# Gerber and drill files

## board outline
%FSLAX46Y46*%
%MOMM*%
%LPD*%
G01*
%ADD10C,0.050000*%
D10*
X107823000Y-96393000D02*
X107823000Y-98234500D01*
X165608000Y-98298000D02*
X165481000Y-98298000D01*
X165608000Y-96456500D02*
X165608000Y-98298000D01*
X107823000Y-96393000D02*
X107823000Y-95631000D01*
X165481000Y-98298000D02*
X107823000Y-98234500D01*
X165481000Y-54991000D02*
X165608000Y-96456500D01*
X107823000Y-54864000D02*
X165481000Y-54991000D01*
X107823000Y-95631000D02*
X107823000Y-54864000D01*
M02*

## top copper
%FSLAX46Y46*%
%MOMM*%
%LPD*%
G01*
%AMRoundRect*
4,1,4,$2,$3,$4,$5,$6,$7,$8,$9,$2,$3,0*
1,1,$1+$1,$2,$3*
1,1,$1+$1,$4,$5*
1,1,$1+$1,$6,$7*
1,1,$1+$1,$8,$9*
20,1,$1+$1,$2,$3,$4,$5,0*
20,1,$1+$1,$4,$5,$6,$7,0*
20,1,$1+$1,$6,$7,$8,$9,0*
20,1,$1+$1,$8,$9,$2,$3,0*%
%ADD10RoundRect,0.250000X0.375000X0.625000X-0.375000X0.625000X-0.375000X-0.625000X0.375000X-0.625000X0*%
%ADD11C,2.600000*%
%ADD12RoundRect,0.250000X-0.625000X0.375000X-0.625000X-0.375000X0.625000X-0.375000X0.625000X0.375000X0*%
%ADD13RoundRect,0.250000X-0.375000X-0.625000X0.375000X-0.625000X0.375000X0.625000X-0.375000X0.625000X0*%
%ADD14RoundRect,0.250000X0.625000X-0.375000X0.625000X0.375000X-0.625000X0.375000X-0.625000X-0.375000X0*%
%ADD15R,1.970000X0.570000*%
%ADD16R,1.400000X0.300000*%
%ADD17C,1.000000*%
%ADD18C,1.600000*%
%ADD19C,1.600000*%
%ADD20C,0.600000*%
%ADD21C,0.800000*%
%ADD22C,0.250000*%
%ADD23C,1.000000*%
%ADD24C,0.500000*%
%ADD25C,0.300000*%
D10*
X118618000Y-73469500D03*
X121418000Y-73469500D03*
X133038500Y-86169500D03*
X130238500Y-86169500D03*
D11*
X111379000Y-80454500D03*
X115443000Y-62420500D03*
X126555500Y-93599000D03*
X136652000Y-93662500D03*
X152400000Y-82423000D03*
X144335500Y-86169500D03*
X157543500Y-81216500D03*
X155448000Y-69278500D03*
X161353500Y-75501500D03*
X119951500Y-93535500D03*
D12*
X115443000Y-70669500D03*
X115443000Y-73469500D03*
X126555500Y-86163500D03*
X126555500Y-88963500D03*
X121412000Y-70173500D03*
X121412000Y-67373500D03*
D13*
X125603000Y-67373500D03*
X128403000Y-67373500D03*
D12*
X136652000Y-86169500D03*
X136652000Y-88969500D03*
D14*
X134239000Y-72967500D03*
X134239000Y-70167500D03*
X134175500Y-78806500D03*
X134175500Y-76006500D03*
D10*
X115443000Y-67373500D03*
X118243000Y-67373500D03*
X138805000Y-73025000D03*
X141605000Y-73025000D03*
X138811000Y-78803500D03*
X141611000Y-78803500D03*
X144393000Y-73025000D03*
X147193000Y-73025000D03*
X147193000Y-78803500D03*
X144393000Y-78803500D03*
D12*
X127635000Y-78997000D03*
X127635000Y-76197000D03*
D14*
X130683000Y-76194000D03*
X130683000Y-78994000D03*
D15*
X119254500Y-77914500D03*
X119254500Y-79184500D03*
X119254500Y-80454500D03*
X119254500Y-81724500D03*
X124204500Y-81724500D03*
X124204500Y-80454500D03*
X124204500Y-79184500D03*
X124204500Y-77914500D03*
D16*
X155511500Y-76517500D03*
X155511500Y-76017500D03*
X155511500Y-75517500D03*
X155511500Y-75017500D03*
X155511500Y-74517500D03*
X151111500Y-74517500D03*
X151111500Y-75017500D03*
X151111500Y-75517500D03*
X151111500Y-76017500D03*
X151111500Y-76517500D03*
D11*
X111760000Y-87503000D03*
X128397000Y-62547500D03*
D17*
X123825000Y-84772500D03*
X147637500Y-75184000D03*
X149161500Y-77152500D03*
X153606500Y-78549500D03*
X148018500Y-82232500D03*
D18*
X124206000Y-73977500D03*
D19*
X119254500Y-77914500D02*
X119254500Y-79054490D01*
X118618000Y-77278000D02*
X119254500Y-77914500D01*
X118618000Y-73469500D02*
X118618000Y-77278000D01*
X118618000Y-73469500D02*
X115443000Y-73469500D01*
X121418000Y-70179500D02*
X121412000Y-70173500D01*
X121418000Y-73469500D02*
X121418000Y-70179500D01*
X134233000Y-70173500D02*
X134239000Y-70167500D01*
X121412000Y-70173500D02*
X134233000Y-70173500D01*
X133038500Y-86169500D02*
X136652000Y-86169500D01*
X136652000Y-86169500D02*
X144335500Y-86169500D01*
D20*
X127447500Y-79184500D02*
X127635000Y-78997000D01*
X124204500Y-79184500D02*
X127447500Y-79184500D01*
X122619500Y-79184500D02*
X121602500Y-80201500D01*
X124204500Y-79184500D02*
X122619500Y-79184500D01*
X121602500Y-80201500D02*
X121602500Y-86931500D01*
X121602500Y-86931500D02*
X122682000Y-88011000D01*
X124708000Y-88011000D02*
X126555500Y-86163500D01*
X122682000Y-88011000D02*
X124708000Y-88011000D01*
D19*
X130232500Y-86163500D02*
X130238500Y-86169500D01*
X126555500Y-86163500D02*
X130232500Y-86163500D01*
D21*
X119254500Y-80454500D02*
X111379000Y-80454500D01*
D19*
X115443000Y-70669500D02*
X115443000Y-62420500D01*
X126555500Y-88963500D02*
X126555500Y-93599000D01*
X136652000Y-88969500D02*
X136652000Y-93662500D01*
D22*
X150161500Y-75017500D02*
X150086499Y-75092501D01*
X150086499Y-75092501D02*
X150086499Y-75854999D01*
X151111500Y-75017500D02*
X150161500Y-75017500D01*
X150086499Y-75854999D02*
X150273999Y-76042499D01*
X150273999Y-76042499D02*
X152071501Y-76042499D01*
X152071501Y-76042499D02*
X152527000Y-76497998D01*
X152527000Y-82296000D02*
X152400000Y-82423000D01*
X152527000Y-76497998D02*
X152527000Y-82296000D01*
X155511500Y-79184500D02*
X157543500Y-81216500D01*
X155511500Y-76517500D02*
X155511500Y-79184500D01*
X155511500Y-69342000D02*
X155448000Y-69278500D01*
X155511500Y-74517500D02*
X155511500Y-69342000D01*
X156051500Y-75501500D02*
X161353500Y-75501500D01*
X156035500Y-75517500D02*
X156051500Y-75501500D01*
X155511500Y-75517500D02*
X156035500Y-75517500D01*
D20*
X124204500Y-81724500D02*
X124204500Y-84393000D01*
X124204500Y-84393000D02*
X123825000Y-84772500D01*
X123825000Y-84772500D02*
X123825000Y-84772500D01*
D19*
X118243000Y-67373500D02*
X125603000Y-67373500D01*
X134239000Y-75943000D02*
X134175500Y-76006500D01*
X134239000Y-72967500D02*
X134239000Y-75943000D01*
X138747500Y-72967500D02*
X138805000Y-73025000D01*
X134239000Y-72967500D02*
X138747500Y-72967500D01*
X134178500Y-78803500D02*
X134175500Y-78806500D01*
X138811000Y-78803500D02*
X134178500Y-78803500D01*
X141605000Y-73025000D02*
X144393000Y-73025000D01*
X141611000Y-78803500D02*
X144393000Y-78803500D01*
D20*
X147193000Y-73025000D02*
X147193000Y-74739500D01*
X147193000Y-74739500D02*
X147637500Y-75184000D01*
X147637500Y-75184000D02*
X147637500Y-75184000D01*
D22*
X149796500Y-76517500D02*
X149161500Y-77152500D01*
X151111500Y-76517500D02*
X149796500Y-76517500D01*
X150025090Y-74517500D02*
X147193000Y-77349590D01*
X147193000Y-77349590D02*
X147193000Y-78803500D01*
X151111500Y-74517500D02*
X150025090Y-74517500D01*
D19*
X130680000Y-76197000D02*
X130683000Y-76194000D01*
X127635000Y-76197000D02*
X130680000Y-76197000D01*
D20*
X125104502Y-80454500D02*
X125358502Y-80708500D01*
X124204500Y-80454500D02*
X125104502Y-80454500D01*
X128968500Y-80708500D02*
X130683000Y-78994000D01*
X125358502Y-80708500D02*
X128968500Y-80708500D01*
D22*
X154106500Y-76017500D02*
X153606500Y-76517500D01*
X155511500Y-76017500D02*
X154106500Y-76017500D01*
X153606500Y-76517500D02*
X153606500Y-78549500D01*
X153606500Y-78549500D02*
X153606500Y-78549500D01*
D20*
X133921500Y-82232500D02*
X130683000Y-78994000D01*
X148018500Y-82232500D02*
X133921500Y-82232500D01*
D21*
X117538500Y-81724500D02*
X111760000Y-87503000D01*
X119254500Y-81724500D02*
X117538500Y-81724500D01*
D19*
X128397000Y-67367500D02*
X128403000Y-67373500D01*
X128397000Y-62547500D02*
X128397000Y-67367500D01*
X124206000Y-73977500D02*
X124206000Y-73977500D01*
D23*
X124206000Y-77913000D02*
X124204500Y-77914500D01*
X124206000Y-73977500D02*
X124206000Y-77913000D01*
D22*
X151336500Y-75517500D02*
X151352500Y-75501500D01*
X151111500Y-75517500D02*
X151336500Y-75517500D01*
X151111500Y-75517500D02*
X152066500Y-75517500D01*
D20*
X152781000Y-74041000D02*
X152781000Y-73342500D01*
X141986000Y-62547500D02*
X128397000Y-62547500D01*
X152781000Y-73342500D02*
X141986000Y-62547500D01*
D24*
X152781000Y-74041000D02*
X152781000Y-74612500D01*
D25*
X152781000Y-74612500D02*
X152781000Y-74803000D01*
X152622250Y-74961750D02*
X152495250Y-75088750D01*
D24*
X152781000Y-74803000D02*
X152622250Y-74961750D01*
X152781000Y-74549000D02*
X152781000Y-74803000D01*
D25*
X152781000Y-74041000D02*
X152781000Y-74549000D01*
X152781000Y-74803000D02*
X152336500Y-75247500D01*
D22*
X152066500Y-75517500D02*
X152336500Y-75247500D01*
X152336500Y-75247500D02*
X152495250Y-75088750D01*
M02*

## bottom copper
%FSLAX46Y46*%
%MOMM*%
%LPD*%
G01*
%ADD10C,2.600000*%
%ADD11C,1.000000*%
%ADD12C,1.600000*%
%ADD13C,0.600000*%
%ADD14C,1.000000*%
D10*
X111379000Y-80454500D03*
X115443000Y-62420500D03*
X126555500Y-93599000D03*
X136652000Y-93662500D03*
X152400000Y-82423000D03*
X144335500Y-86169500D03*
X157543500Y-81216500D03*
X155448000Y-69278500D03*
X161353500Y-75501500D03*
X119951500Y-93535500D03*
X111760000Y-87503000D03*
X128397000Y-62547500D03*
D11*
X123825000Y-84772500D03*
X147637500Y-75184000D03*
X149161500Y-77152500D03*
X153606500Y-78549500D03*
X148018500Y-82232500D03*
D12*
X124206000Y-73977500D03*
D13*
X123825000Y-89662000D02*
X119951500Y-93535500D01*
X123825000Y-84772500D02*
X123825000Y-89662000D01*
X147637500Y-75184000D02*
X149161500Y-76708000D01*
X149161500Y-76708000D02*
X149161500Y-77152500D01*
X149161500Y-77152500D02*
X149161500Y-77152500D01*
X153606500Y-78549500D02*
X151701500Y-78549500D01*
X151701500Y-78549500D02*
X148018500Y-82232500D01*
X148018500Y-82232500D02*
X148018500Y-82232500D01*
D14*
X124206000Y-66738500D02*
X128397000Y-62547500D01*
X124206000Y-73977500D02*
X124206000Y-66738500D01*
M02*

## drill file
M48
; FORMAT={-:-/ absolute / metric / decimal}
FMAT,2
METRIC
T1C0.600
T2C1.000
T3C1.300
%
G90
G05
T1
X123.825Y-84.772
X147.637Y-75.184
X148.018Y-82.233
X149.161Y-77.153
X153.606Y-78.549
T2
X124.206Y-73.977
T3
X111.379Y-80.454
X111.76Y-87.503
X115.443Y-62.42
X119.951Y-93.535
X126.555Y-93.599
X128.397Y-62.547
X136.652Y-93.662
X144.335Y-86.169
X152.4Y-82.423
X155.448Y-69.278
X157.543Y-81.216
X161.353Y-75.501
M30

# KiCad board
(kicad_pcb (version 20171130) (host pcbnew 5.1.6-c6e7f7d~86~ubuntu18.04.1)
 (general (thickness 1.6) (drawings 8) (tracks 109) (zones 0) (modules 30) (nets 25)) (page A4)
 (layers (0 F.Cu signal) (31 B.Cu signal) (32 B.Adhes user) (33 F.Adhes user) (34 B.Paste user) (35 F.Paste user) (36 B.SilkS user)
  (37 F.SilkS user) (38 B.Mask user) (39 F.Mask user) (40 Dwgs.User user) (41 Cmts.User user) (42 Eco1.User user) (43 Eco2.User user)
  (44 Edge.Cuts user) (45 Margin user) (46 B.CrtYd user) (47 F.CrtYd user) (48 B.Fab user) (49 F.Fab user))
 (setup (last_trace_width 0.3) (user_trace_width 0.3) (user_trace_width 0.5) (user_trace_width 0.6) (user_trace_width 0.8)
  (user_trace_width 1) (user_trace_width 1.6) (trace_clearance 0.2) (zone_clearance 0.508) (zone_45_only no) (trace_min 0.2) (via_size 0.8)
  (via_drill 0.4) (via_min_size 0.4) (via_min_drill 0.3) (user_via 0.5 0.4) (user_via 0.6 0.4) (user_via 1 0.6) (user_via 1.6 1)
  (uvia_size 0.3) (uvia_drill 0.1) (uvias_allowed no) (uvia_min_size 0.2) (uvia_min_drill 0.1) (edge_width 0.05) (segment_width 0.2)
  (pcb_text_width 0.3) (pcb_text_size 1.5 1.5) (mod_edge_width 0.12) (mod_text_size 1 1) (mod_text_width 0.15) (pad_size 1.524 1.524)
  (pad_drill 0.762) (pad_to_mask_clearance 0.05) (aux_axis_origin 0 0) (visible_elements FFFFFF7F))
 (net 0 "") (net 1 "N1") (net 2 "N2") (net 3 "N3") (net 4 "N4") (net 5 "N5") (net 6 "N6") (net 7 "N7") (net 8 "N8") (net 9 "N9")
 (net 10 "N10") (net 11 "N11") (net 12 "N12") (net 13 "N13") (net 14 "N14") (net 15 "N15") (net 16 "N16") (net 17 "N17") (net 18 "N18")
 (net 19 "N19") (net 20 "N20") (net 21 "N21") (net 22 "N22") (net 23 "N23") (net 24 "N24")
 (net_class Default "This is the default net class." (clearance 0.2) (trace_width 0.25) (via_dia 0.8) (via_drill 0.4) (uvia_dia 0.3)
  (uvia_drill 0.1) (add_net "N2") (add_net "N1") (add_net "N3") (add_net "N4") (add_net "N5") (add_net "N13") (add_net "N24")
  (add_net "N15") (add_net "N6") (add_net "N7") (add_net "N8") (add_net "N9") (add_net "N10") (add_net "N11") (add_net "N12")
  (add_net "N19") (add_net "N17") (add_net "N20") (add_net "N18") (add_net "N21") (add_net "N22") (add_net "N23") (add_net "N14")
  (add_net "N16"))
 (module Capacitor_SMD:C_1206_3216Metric (layer F.Cu) (at 120.018 73.4695 180)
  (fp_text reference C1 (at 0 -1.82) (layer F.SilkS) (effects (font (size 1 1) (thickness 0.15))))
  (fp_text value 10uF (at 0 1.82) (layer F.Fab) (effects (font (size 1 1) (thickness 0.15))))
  (pad 2 smd roundrect (at 1.4 0 180) (size 1.25 1.75) (layers F.Cu F.Paste F.Mask) (roundrect_rratio 0.2) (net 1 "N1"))
  (pad 1 smd roundrect (at -1.4 0 180) (size 1.25 1.75) (layers F.Cu F.Paste F.Mask) (roundrect_rratio 0.2) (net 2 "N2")))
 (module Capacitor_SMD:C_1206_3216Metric (layer F.Cu) (at 131.6385 86.1695 180)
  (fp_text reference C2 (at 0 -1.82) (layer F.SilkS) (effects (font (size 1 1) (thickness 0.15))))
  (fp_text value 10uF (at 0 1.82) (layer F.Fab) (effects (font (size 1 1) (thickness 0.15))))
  (pad 1 smd roundrect (at -1.4 0 180) (size 1.25 1.75) (layers F.Cu F.Paste F.Mask) (roundrect_rratio 0.2) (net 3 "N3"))
  (pad 2 smd roundrect (at 1.4 0 180) (size 1.25 1.75) (layers F.Cu F.Paste F.Mask) (roundrect_rratio 0.2) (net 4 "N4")))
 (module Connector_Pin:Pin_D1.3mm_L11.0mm (layer F.Cu) (at 111.379 80.4545)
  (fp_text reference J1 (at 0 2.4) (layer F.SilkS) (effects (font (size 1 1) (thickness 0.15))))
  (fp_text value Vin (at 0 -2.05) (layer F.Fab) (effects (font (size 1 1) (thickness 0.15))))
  (pad 1 thru_hole circle (at 0 0) (size 2.6 2.6) (drill 1.3) (layers *.Cu *.Mask) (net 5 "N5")))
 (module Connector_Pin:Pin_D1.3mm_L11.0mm (layer F.Cu) (at 115.443 62.4205)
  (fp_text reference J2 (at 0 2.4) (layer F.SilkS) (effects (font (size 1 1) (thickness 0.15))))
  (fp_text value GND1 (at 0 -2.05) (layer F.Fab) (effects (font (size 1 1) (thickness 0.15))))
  (pad 1 thru_hole circle (at 0 0) (size 2.6 2.6) (drill 1.3) (layers *.Cu *.Mask) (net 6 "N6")))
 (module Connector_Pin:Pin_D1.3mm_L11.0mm (layer F.Cu) (at 126.5555 93.599)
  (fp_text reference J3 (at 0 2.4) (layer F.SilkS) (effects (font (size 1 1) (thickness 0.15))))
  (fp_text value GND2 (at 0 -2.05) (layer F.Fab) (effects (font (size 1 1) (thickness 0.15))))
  (pad 1 thru_hole circle (at 0 0) (size 2.6 2.6) (drill 1.3) (layers *.Cu *.Mask) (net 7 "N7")))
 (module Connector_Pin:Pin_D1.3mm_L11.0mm (layer F.Cu) (at 136.652 93.6625)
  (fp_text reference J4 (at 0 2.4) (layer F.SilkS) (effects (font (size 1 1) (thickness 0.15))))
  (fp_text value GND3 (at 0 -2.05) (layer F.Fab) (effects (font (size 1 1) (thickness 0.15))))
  (pad 1 thru_hole circle (at 0 0) (size 2.6 2.6) (drill 1.3) (layers *.Cu *.Mask) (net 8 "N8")))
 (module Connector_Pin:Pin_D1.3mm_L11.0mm (layer F.Cu) (at 152.4 82.423)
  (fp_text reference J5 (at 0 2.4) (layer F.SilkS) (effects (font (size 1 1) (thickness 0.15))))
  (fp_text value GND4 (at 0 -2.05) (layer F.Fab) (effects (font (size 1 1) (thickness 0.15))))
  (pad 1 thru_hole circle (at 0 0) (size 2.6 2.6) (drill 1.3) (layers *.Cu *.Mask) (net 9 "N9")))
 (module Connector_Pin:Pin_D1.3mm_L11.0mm (layer F.Cu) (at 144.3355 86.1695)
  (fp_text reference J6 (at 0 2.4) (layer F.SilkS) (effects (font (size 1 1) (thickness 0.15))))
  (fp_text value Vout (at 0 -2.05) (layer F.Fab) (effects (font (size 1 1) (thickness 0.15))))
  (pad 1 thru_hole circle (at 0 0) (size 2.6 2.6) (drill 1.3) (layers *.Cu *.Mask) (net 3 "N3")))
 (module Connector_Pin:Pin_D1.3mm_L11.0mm (layer F.Cu) (at 157.5435 81.2165)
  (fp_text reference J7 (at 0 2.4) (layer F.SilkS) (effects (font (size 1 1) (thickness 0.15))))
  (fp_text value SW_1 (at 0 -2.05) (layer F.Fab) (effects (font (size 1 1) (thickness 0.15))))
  (pad 1 thru_hole circle (at 0 0) (size 2.6 2.6) (drill 1.3) (layers *.Cu *.Mask) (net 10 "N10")))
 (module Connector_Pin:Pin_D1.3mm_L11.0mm (layer F.Cu) (at 155.448 69.2785)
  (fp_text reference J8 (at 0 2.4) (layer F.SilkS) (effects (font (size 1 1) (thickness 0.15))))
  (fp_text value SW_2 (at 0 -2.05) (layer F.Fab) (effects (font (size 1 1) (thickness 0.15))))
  (pad 1 thru_hole circle (at 0 0) (size 2.6 2.6) (drill 1.3) (layers *.Cu *.Mask) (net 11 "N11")))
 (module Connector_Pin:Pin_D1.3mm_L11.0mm (layer F.Cu) (at 161.3535 75.5015)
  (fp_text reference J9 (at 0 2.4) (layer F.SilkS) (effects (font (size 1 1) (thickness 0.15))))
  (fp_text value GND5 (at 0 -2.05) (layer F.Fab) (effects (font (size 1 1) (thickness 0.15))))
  (pad 1 thru_hole circle (at 0 0) (size 2.6 2.6) (drill 1.3) (layers *.Cu *.Mask) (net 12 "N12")))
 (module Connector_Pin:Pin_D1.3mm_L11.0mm (layer F.Cu) (at 119.9515 93.5355)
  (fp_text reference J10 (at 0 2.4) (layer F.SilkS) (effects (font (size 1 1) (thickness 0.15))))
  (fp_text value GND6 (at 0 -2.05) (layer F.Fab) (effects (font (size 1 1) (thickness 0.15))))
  (pad 1 thru_hole circle (at 0 0) (size 2.6 2.6) (drill 1.3) (layers *.Cu *.Mask) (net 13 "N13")))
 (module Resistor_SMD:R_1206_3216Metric (layer F.Cu) (at 115.443 72.0695 270)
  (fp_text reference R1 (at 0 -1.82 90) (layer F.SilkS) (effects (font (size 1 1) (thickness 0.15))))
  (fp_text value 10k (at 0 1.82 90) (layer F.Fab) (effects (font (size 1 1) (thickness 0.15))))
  (pad 1 smd roundrect (at -1.4 0 270) (size 1.25 1.75) (layers F.Cu F.Paste F.Mask) (roundrect_rratio 0.2) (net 6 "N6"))
  (pad 2 smd roundrect (at 1.4 0 270) (size 1.25 1.75) (layers F.Cu F.Paste F.Mask) (roundrect_rratio 0.2) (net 1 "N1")))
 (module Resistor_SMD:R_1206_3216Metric (layer F.Cu) (at 126.5555 87.5635 270)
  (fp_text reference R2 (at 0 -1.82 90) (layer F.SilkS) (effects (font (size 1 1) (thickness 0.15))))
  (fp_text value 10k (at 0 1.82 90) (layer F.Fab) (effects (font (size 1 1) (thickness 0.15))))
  (pad 1 smd roundrect (at -1.4 0 270) (size 1.25 1.75) (layers F.Cu F.Paste F.Mask) (roundrect_rratio 0.2) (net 4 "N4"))
  (pad 2 smd roundrect (at 1.4 0 270) (size 1.25 1.75) (layers F.Cu F.Paste F.Mask) (roundrect_rratio 0.2) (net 7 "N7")))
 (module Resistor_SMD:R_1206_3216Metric (layer F.Cu) (at 121.412 68.7735 270)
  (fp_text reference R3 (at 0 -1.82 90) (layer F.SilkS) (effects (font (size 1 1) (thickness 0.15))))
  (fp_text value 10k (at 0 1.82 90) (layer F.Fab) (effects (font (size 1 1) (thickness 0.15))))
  (pad 2 smd roundrect (at 1.4 0 270) (size 1.25 1.75) (layers F.Cu F.Paste F.Mask) (roundrect_rratio 0.2) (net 2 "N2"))
  (pad 1 smd roundrect (at -1.4 0 270) (size 1.25 1.75) (layers F.Cu F.Paste F.Mask) (roundrect_rratio 0.2) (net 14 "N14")))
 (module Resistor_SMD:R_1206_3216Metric (layer F.Cu) (at 127.003 67.3735)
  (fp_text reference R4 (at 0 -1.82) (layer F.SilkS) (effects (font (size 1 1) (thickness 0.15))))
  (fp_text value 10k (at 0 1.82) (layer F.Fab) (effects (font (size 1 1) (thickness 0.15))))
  (pad 1 smd roundrect (at -1.4 0) (size 1.25 1.75) (layers F.Cu F.Paste F.Mask) (roundrect_rratio 0.2) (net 14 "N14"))
  (pad 2 smd roundrect (at 1.4 0) (size 1.25 1.75) (layers F.Cu F.Paste F.Mask) (roundrect_rratio 0.2) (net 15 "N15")))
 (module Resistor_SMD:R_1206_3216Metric (layer F.Cu) (at 136.652 87.5695 270)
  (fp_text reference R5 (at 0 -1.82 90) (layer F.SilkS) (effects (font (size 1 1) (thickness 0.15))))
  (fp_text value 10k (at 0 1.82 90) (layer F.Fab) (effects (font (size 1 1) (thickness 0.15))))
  (pad 1 smd roundrect (at -1.4 0 270) (size 1.25 1.75) (layers F.Cu F.Paste F.Mask) (roundrect_rratio 0.2) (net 3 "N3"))
  (pad 2 smd roundrect (at 1.4 0 270) (size 1.25 1.75) (layers F.Cu F.Paste F.Mask) (roundrect_rratio 0.2) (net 8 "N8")))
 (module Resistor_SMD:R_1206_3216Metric (layer F.Cu) (at 134.239 71.5675 90)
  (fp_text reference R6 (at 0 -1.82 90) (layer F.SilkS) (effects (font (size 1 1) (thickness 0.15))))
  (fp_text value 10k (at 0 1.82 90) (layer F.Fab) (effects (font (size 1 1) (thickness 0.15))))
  (pad 1 smd roundrect (at -1.4 0 90) (size 1.25 1.75) (layers F.Cu F.Paste F.Mask) (roundrect_rratio 0.2) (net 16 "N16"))
  (pad 2 smd roundrect (at 1.4 0 90) (size 1.25 1.75) (layers F.Cu F.Paste F.Mask) (roundrect_rratio 0.2) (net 2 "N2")))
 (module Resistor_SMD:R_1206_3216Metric (layer F.Cu) (at 134.1755 77.4065 90)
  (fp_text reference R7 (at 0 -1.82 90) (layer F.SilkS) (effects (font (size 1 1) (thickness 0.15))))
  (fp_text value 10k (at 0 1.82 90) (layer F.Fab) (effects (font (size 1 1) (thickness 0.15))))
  (pad 1 smd roundrect (at -1.4 0 90) (size 1.25 1.75) (layers F.Cu F.Paste F.Mask) (roundrect_rratio 0.2) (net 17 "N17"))
  (pad 2 smd roundrect (at 1.4 0 90) (size 1.25 1.75) (layers F.Cu F.Paste F.Mask) (roundrect_rratio 0.2) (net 16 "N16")))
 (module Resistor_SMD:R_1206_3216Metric (layer F.Cu) (at 116.843 67.3735 180)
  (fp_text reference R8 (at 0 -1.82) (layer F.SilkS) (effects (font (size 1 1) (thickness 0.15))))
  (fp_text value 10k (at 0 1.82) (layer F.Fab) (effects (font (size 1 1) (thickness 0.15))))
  (pad 2 smd roundrect (at 1.4 0 180) (size 1.25 1.75) (layers F.Cu F.Paste F.Mask) (roundrect_rratio 0.2) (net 6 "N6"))
  (pad 1 smd roundrect (at -1.4 0 180) (size 1.25 1.75) (layers F.Cu F.Paste F.Mask) (roundrect_rratio 0.2) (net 14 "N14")))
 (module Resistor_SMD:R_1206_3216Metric (layer F.Cu) (at 140.205 73.025 180)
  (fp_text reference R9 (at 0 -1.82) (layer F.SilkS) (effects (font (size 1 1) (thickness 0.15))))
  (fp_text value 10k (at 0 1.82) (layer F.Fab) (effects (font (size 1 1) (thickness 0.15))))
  (pad 2 smd roundrect (at 1.4 0 180) (size 1.25 1.75) (layers F.Cu F.Paste F.Mask) (roundrect_rratio 0.2) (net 16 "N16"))
  (pad 1 smd roundrect (at -1.4 0 180) (size 1.25 1.75) (layers F.Cu F.Paste F.Mask) (roundrect_rratio 0.2) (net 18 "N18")))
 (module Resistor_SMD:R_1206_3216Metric (layer F.Cu) (at 140.211 78.8035 180)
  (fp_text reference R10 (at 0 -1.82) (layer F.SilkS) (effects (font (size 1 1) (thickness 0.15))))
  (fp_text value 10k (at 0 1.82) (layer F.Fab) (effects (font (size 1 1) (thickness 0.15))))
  (pad 2 smd roundrect (at 1.4 0 180) (size 1.25 1.75) (layers F.Cu F.Paste F.Mask) (roundrect_rratio 0.2) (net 17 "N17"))
  (pad 1 smd roundrect (at -1.4 0 180) (size 1.25 1.75) (layers F.Cu F.Paste F.Mask) (roundrect_rratio 0.2) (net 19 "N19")))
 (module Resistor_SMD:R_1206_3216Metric (layer F.Cu) (at 145.793 73.025 180)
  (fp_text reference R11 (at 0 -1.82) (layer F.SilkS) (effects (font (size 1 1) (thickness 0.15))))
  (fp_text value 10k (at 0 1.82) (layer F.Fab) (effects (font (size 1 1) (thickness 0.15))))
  (pad 2 smd roundrect (at 1.4 0 180) (size 1.25 1.75) (layers F.Cu F.Paste F.Mask) (roundrect_rratio 0.2) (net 18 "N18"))
  (pad 1 smd roundrect (at -1.4 0 180) (size 1.25 1.75) (layers F.Cu F.Paste F.Mask) (roundrect_rratio 0.2) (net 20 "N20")))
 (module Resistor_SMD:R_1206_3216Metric (layer F.Cu) (at 145.793 78.8035 180)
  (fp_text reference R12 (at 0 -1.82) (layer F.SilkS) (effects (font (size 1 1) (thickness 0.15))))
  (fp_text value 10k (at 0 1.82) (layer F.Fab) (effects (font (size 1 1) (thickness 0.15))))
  (pad 1 smd roundrect (at -1.4 0 180) (size 1.25 1.75) (layers F.Cu F.Paste F.Mask) (roundrect_rratio 0.2) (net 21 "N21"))
  (pad 2 smd roundrect (at 1.4 0 180) (size 1.25 1.75) (layers F.Cu F.Paste F.Mask) (roundrect_rratio 0.2) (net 19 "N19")))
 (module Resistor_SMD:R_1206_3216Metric (layer F.Cu) (at 127.635 77.597 270)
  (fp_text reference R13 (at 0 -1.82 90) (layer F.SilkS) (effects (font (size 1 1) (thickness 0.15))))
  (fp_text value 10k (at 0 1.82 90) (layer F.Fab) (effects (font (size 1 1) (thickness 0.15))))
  (pad 2 smd roundrect (at 1.4 0 270) (size 1.25 1.75) (layers F.Cu F.Paste F.Mask) (roundrect_rratio 0.2) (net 4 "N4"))
  (pad 1 smd roundrect (at -1.4 0 270) (size 1.25 1.75) (layers F.Cu F.Paste F.Mask) (roundrect_rratio 0.2) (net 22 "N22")))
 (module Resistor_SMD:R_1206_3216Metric (layer F.Cu) (at 130.683 77.594 90)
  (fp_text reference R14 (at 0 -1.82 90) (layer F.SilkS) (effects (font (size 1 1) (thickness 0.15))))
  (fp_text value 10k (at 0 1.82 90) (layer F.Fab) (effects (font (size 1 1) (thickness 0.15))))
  (pad 2 smd roundrect (at 1.4 0 90) (size 1.25 1.75) (layers F.Cu F.Paste F.Mask) (roundrect_rratio 0.2) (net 22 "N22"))
  (pad 1 smd roundrect (at -1.4 0 90) (size 1.25 1.75) (layers F.Cu F.Paste F.Mask) (roundrect_rratio 0.2) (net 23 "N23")))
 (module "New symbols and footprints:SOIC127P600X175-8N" (layer F.Cu) (at 121.7295 79.8195)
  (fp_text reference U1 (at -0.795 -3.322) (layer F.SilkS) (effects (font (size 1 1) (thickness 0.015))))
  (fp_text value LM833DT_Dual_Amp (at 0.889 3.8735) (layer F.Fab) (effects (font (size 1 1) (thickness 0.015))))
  (pad 1 smd rect (at -2.475 -1.905) (size 1.97 0.57) (layers F.Cu F.Paste F.Mask) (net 1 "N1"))
  (pad 2 smd rect (at -2.475 -0.635) (size 1.97 0.57) (layers F.Cu F.Paste F.Mask) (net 1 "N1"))
  (pad 3 smd rect (at -2.475 0.635) (size 1.97 0.57) (layers F.Cu F.Paste F.Mask) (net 5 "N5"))
  (pad 4 smd rect (at -2.475 1.905) (size 1.97 0.57) (layers F.Cu F.Paste F.Mask) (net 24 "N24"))
  (pad 5 smd rect (at 2.475 1.905) (size 1.97 0.57) (layers F.Cu F.Paste F.Mask) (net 13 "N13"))
  (pad 6 smd rect (at 2.475 0.635) (size 1.97 0.57) (layers F.Cu F.Paste F.Mask) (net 23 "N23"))
  (pad 7 smd rect (at 2.475 -0.635) (size 1.97 0.57) (layers F.Cu F.Paste F.Mask) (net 4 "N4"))
  (pad 8 smd rect (at 2.475 -1.905) (size 1.97 0.57) (layers F.Cu F.Paste F.Mask) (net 15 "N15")))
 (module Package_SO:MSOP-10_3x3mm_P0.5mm (layer F.Cu) (at 153.3115 75.5175 180)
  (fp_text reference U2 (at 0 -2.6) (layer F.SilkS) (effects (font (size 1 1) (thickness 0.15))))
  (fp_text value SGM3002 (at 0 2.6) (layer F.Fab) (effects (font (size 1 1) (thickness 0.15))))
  (pad 1 smd rect (at -2.2 -1 180) (size 1.4 0.3) (layers F.Cu F.Paste F.Mask) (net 10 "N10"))
  (pad 2 smd rect (at -2.2 -0.5 180) (size 1.4 0.3) (layers F.Cu F.Paste F.Mask) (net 23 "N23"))
  (pad 3 smd rect (at -2.2 0 180) (size 1.4 0.3) (layers F.Cu F.Paste F.Mask) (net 12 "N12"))
  (pad 4 smd rect (at -2.2 0.5 180) (size 1.4 0.3) (layers F.Cu F.Paste F.Mask) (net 23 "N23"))
  (pad 5 smd rect (at -2.2 1 180) (size 1.4 0.3) (layers F.Cu F.Paste F.Mask) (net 11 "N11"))
  (pad 6 smd rect (at 2.2 1 180) (size 1.4 0.3) (layers F.Cu F.Paste F.Mask) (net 21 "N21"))
  (pad 7 smd rect (at 2.2 0.5 180) (size 1.4 0.3) (layers F.Cu F.Paste F.Mask) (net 9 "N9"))
  (pad 8 smd rect (at 2.2 0 180) (size 1.4 0.3) (layers F.Cu F.Paste F.Mask) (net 15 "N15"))
  (pad 9 smd rect (at 2.2 -0.5 180) (size 1.4 0.3) (layers F.Cu F.Paste F.Mask) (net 9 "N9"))
  (pad 10 smd rect (at 2.2 -1 180) (size 1.4 0.3) (layers F.Cu F.Paste F.Mask) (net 20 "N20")))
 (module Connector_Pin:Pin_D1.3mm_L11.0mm (layer F.Cu) (at 111.76 87.503)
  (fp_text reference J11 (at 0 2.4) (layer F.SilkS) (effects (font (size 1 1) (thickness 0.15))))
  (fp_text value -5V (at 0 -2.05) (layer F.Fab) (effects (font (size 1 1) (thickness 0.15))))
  (pad 1 thru_hole circle (at 0 0) (size 2.6 2.6) (drill 1.3) (layers *.Cu *.Mask) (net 24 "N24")))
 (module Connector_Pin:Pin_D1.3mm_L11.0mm (layer F.Cu) (at 128.397 62.5475)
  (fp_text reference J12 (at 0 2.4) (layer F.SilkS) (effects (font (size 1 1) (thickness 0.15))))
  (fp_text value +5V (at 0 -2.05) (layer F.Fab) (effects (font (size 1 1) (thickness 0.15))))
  (pad 1 thru_hole circle (at 0 0) (size 2.6 2.6) (drill 1.3) (layers *.Cu *.Mask) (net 15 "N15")))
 (gr_line (start 107.823 96.393) (end 107.823 98.2345) (layer Edge.Cuts) (width 0.05))
 (gr_line (start 165.608 98.298) (end 165.481 98.298) (layer Edge.Cuts) (width 0.05))
 (gr_line (start 165.608 96.4565) (end 165.608 98.298) (layer Edge.Cuts) (width 0.05))
 (gr_line (start 107.823 96.393) (end 107.823 95.631) (layer Edge.Cuts) (width 0.05))
 (gr_line (start 165.481 98.298) (end 107.823 98.2345) (layer Edge.Cuts) (width 0.05))
 (gr_line (start 165.481 54.991) (end 165.608 96.4565) (layer Edge.Cuts) (width 0.05))
 (gr_line (start 107.823 54.864) (end 165.481 54.991) (layer Edge.Cuts) (width 0.05))
 (gr_line (start 107.823 95.631) (end 107.823 54.864) (layer Edge.Cuts) (width 0.05))
 (segment (start 119.2545 77.9145) (end 119.2545 79.05449) (width 1.6) (layer F.Cu) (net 1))
 (segment (start 118.618 77.278) (end 119.2545 77.9145) (width 1.6) (layer F.Cu) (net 1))
 (segment (start 118.618 73.4695) (end 118.618 77.278) (width 1.6) (layer F.Cu) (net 1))
 (segment (start 118.618 73.4695) (end 115.443 73.4695) (width 1.6) (layer F.Cu) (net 1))
 (segment (start 121.418 70.1795) (end 121.412 70.1735) (width 1.6) (layer F.Cu) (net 2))
 (segment (start 121.418 73.4695) (end 121.418 70.1795) (width 1.6) (layer F.Cu) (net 2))
 (segment (start 134.233 70.1735) (end 134.239 70.1675) (width 1.6) (layer F.Cu) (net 2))
 (segment (start 121.412 70.1735) (end 134.233 70.1735) (width 1.6) (layer F.Cu) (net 2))
 (segment (start 133.0385 86.1695) (end 136.652 86.1695) (width 1.6) (layer F.Cu) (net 3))
 (segment (start 136.652 86.1695) (end 144.3355 86.1695) (width 1.6) (layer F.Cu) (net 3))
 (segment (start 127.4475 79.1845) (end 127.635 78.997) (width 0.6) (layer F.Cu) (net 4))
 (segment (start 124.2045 79.1845) (end 127.4475 79.1845) (width 0.6) (layer F.Cu) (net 4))
 (segment (start 122.6195 79.1845) (end 121.6025 80.2015) (width 0.6) (layer F.Cu) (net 4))
 (segment (start 124.2045 79.1845) (end 122.6195 79.1845) (width 0.6) (layer F.Cu) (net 4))
 (segment (start 121.6025 80.2015) (end 121.6025 86.9315) (width 0.6) (layer F.Cu) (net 4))
 (segment (start 121.6025 86.9315) (end 122.682 88.011) (width 0.6) (layer F.Cu) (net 4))
 (segment (start 124.708 88.011) (end 126.5555 86.1635) (width 0.6) (layer F.Cu) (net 4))
 (segment (start 122.682 88.011) (end 124.708 88.011) (width 0.6) (layer F.Cu) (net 4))
 (segment (start 130.2325 86.1635) (end 130.2385 86.1695) (width 1.6) (layer F.Cu) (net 4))
 (segment (start 126.5555 86.1635) (end 130.2325 86.1635) (width 1.6) (layer F.Cu) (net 4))
 (segment (start 119.2545 80.4545) (end 111.379 80.4545) (width 0.8) (layer F.Cu) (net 5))
 (segment (start 115.443 70.6695) (end 115.443 62.4205) (width 1.6) (layer F.Cu) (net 6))
 (segment (start 126.5555 88.9635) (end 126.5555 93.599) (width 1.6) (layer F.Cu) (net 7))
 (segment (start 136.652 88.9695) (end 136.652 93.6625) (width 1.6) (layer F.Cu) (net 8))
 (segment (start 150.1615 75.0175) (end 150.086499 75.092501) (width 0.25) (layer F.Cu) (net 9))
 (segment (start 150.086499 75.092501) (end 150.086499 75.854999) (width 0.25) (layer F.Cu) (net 9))
 (segment (start 151.1115 75.0175) (end 150.1615 75.0175) (width 0.25) (layer F.Cu) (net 9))
 (segment (start 150.086499 75.854999) (end 150.273999 76.042499) (width 0.25) (layer F.Cu) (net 9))
 (segment (start 150.273999 76.042499) (end 152.071501 76.042499) (width 0.25) (layer F.Cu) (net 9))
 (segment (start 152.071501 76.042499) (end 152.527 76.497998) (width 0.25) (layer F.Cu) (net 9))
 (segment (start 152.527 82.296) (end 152.4 82.423) (width 0.25) (layer F.Cu) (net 9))
 (segment (start 152.527 76.497998) (end 152.527 82.296) (width 0.25) (layer F.Cu) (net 9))
 (segment (start 155.5115 79.1845) (end 157.5435 81.2165) (width 0.25) (layer F.Cu) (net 10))
 (segment (start 155.5115 76.5175) (end 155.5115 79.1845) (width 0.25) (layer F.Cu) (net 10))
 (segment (start 155.5115 69.342) (end 155.448 69.2785) (width 0.25) (layer F.Cu) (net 11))
 (segment (start 155.5115 74.5175) (end 155.5115 69.342) (width 0.25) (layer F.Cu) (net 11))
 (segment (start 156.0515 75.5015) (end 161.3535 75.5015) (width 0.25) (layer F.Cu) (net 12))
 (segment (start 156.0355 75.5175) (end 156.0515 75.5015) (width 0.25) (layer F.Cu) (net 12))
 (segment (start 155.5115 75.5175) (end 156.0355 75.5175) (width 0.25) (layer F.Cu) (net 12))
 (segment (start 124.2045 81.7245) (end 124.2045 84.393) (width 0.6) (layer F.Cu) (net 13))
 (segment (start 124.2045 84.393) (end 123.825 84.7725) (width 0.6) (layer F.Cu) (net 13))
 (segment (start 123.825 84.7725) (end 123.825 84.7725) (width 0.6) (layer F.Cu) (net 13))
 (via (at 123.825 84.7725) (size 1) (drill 0.6) (layers F.Cu B.Cu) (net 13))
 (segment (start 123.825 89.662) (end 119.9515 93.5355) (width 0.6) (layer B.Cu) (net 13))
 (segment (start 123.825 84.7725) (end 123.825 89.662) (width 0.6) (layer B.Cu) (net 13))
 (segment (start 118.243 67.3735) (end 125.603 67.3735) (width 1.6) (layer F.Cu) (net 14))
 (segment (start 134.239 75.943) (end 134.1755 76.0065) (width 1.6) (layer F.Cu) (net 16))
 (segment (start 134.239 72.9675) (end 134.239 75.943) (width 1.6) (layer F.Cu) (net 16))
 (segment (start 138.7475 72.9675) (end 138.805 73.025) (width 1.6) (layer F.Cu) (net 16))
 (segment (start 134.239 72.9675) (end 138.7475 72.9675) (width 1.6) (layer F.Cu) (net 16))
 (segment (start 134.1785 78.8035) (end 134.1755 78.8065) (width 1.6) (layer F.Cu) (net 17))
 (segment (start 138.811 78.8035) (end 134.1785 78.8035) (width 1.6) (layer F.Cu) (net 17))
 (segment (start 141.605 73.025) (end 144.393 73.025) (width 1.6) (layer F.Cu) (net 18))
 (segment (start 141.611 78.8035) (end 144.393 78.8035) (width 1.6) (layer F.Cu) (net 19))
 (segment (start 147.193 73.025) (end 147.193 74.7395) (width 0.6) (layer F.Cu) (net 20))
 (segment (start 147.193 74.7395) (end 147.6375 75.184) (width 0.6) (layer F.Cu) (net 20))
 (segment (start 147.6375 75.184) (end 147.6375 75.184) (width 0.6) (layer F.Cu) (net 20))
 (via (at 147.6375 75.184) (size 1) (drill 0.6) (layers F.Cu B.Cu) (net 20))
 (segment (start 147.6375 75.184) (end 149.1615 76.708) (width 0.6) (layer B.Cu) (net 20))
 (segment (start 149.1615 76.708) (end 149.1615 77.1525) (width 0.6) (layer B.Cu) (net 20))
 (segment (start 149.1615 77.1525) (end 149.1615 77.1525) (width 0.6) (layer B.Cu) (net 20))
 (via (at 149.1615 77.1525) (size 1) (drill 0.6) (layers F.Cu B.Cu) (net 20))
 (segment (start 149.7965 76.5175) (end 149.1615 77.1525) (width 0.25) (layer F.Cu) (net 20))
 (segment (start 151.1115 76.5175) (end 149.7965 76.5175) (width 0.25) (layer F.Cu) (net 20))
 (segment (start 150.02509 74.5175) (end 147.193 77.34959) (width 0.25) (layer F.Cu) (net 21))
 (segment (start 147.193 77.34959) (end 147.193 78.8035) (width 0.25) (layer F.Cu) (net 21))
 (segment (start 151.1115 74.5175) (end 150.02509 74.5175) (width 0.25) (layer F.Cu) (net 21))
 (segment (start 130.68 76.197) (end 130.683 76.194) (width 1.6) (layer F.Cu) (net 22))
 (segment (start 127.635 76.197) (end 130.68 76.197) (width 1.6) (layer F.Cu) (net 22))
 (segment (start 125.104502 80.4545) (end 125.358502 80.7085) (width 0.6) (layer F.Cu) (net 23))
 (segment (start 124.2045 80.4545) (end 125.104502 80.4545) (width 0.6) (layer F.Cu) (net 23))
 (segment (start 128.9685 80.7085) (end 130.683 78.994) (width 0.6) (layer F.Cu) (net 23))
 (segment (start 125.358502 80.7085) (end 128.9685 80.7085) (width 0.6) (layer F.Cu) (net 23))
 (segment (start 154.1065 76.0175) (end 153.6065 76.5175) (width 0.25) (layer F.Cu) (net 23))
 (segment (start 155.5115 76.0175) (end 154.1065 76.0175) (width 0.25) (layer F.Cu) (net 23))
 (segment (start 153.6065 76.5175) (end 153.6065 78.5495) (width 0.25) (layer F.Cu) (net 23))
 (segment (start 153.6065 78.5495) (end 153.6065 78.5495) (width 0.25) (layer F.Cu) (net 23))
 (via (at 153.6065 78.5495) (size 1) (drill 0.6) (layers F.Cu B.Cu) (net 23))
 (segment (start 153.6065 78.5495) (end 151.7015 78.5495) (width 0.6) (layer B.Cu) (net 23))
 (segment (start 151.7015 78.5495) (end 148.0185 82.2325) (width 0.6) (layer B.Cu) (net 23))
 (segment (start 148.0185 82.2325) (end 148.0185 82.2325) (width 0.6) (layer B.Cu) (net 23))
 (via (at 148.0185 82.2325) (size 1) (drill 0.6) (layers F.Cu B.Cu) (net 23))
 (segment (start 133.9215 82.2325) (end 130.683 78.994) (width 0.6) (layer F.Cu) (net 23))
 (segment (start 148.0185 82.2325) (end 133.9215 82.2325) (width 0.6) (layer F.Cu) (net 23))
 (segment (start 117.5385 81.7245) (end 111.76 87.503) (width 0.8) (layer F.Cu) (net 24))
 (segment (start 119.2545 81.7245) (end 117.5385 81.7245) (width 0.8) (layer F.Cu) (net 24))
 (segment (start 128.397 67.3675) (end 128.403 67.3735) (width 1.6) (layer F.Cu) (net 15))
 (segment (start 128.397 62.5475) (end 128.397 67.3675) (width 1.6) (layer F.Cu) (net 15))
 (segment (start 124.206 73.9775) (end 124.206 73.9775) (width 1.6) (layer F.Cu) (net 15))
 (via (at 124.206 73.9775) (size 1.6) (drill 1) (layers F.Cu B.Cu) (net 15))
 (segment (start 124.206 77.913) (end 124.2045 77.9145) (width 1) (layer F.Cu) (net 15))
 (segment (start 124.206 73.9775) (end 124.206 77.913) (width 1) (layer F.Cu) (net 15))
 (segment (start 124.206 66.7385) (end 128.397 62.5475) (width 1) (layer B.Cu) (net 15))
 (segment (start 124.206 73.9775) (end 124.206 66.7385) (width 1) (layer B.Cu) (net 15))
 (segment (start 151.3365 75.5175) (end 151.3525 75.5015) (width 0.25) (layer F.Cu) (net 15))
 (segment (start 151.1115 75.5175) (end 151.3365 75.5175) (width 0.25) (layer F.Cu) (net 15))
 (segment (start 151.1115 75.5175) (end 152.0665 75.5175) (width 0.25) (layer F.Cu) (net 15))
 (segment (start 152.781 74.041) (end 152.781 73.3425) (width 0.6) (layer F.Cu) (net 15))
 (segment (start 141.986 62.5475) (end 128.397 62.5475) (width 0.6) (layer F.Cu) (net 15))
 (segment (start 152.781 73.3425) (end 141.986 62.5475) (width 0.6) (layer F.Cu) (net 15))
 (segment (start 152.781 74.041) (end 152.781 74.6125) (width 0.5) (layer F.Cu) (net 15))
 (segment (start 152.781 74.6125) (end 152.781 74.803) (width 0.3) (layer F.Cu) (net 15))
 (segment (start 152.62225 74.96175) (end 152.49525 75.08875) (width 0.3) (layer F.Cu) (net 15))
 (segment (start 152.781 74.803) (end 152.62225 74.96175) (width 0.5) (layer F.Cu) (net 15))
 (segment (start 152.781 74.549) (end 152.781 74.803) (width 0.5) (layer F.Cu) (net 15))
 (segment (start 152.781 74.041) (end 152.781 74.549) (width 0.3) (layer F.Cu) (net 15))
 (segment (start 152.781 74.803) (end 152.3365 75.2475) (width 0.3) (layer F.Cu) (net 15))
 (segment (start 152.0665 75.5175) (end 152.3365 75.2475) (width 0.25) (layer F.Cu) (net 15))
 (segment (start 152.3365 75.2475) (end 152.49525 75.08875) (width 0.25) (layer F.Cu) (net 15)))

